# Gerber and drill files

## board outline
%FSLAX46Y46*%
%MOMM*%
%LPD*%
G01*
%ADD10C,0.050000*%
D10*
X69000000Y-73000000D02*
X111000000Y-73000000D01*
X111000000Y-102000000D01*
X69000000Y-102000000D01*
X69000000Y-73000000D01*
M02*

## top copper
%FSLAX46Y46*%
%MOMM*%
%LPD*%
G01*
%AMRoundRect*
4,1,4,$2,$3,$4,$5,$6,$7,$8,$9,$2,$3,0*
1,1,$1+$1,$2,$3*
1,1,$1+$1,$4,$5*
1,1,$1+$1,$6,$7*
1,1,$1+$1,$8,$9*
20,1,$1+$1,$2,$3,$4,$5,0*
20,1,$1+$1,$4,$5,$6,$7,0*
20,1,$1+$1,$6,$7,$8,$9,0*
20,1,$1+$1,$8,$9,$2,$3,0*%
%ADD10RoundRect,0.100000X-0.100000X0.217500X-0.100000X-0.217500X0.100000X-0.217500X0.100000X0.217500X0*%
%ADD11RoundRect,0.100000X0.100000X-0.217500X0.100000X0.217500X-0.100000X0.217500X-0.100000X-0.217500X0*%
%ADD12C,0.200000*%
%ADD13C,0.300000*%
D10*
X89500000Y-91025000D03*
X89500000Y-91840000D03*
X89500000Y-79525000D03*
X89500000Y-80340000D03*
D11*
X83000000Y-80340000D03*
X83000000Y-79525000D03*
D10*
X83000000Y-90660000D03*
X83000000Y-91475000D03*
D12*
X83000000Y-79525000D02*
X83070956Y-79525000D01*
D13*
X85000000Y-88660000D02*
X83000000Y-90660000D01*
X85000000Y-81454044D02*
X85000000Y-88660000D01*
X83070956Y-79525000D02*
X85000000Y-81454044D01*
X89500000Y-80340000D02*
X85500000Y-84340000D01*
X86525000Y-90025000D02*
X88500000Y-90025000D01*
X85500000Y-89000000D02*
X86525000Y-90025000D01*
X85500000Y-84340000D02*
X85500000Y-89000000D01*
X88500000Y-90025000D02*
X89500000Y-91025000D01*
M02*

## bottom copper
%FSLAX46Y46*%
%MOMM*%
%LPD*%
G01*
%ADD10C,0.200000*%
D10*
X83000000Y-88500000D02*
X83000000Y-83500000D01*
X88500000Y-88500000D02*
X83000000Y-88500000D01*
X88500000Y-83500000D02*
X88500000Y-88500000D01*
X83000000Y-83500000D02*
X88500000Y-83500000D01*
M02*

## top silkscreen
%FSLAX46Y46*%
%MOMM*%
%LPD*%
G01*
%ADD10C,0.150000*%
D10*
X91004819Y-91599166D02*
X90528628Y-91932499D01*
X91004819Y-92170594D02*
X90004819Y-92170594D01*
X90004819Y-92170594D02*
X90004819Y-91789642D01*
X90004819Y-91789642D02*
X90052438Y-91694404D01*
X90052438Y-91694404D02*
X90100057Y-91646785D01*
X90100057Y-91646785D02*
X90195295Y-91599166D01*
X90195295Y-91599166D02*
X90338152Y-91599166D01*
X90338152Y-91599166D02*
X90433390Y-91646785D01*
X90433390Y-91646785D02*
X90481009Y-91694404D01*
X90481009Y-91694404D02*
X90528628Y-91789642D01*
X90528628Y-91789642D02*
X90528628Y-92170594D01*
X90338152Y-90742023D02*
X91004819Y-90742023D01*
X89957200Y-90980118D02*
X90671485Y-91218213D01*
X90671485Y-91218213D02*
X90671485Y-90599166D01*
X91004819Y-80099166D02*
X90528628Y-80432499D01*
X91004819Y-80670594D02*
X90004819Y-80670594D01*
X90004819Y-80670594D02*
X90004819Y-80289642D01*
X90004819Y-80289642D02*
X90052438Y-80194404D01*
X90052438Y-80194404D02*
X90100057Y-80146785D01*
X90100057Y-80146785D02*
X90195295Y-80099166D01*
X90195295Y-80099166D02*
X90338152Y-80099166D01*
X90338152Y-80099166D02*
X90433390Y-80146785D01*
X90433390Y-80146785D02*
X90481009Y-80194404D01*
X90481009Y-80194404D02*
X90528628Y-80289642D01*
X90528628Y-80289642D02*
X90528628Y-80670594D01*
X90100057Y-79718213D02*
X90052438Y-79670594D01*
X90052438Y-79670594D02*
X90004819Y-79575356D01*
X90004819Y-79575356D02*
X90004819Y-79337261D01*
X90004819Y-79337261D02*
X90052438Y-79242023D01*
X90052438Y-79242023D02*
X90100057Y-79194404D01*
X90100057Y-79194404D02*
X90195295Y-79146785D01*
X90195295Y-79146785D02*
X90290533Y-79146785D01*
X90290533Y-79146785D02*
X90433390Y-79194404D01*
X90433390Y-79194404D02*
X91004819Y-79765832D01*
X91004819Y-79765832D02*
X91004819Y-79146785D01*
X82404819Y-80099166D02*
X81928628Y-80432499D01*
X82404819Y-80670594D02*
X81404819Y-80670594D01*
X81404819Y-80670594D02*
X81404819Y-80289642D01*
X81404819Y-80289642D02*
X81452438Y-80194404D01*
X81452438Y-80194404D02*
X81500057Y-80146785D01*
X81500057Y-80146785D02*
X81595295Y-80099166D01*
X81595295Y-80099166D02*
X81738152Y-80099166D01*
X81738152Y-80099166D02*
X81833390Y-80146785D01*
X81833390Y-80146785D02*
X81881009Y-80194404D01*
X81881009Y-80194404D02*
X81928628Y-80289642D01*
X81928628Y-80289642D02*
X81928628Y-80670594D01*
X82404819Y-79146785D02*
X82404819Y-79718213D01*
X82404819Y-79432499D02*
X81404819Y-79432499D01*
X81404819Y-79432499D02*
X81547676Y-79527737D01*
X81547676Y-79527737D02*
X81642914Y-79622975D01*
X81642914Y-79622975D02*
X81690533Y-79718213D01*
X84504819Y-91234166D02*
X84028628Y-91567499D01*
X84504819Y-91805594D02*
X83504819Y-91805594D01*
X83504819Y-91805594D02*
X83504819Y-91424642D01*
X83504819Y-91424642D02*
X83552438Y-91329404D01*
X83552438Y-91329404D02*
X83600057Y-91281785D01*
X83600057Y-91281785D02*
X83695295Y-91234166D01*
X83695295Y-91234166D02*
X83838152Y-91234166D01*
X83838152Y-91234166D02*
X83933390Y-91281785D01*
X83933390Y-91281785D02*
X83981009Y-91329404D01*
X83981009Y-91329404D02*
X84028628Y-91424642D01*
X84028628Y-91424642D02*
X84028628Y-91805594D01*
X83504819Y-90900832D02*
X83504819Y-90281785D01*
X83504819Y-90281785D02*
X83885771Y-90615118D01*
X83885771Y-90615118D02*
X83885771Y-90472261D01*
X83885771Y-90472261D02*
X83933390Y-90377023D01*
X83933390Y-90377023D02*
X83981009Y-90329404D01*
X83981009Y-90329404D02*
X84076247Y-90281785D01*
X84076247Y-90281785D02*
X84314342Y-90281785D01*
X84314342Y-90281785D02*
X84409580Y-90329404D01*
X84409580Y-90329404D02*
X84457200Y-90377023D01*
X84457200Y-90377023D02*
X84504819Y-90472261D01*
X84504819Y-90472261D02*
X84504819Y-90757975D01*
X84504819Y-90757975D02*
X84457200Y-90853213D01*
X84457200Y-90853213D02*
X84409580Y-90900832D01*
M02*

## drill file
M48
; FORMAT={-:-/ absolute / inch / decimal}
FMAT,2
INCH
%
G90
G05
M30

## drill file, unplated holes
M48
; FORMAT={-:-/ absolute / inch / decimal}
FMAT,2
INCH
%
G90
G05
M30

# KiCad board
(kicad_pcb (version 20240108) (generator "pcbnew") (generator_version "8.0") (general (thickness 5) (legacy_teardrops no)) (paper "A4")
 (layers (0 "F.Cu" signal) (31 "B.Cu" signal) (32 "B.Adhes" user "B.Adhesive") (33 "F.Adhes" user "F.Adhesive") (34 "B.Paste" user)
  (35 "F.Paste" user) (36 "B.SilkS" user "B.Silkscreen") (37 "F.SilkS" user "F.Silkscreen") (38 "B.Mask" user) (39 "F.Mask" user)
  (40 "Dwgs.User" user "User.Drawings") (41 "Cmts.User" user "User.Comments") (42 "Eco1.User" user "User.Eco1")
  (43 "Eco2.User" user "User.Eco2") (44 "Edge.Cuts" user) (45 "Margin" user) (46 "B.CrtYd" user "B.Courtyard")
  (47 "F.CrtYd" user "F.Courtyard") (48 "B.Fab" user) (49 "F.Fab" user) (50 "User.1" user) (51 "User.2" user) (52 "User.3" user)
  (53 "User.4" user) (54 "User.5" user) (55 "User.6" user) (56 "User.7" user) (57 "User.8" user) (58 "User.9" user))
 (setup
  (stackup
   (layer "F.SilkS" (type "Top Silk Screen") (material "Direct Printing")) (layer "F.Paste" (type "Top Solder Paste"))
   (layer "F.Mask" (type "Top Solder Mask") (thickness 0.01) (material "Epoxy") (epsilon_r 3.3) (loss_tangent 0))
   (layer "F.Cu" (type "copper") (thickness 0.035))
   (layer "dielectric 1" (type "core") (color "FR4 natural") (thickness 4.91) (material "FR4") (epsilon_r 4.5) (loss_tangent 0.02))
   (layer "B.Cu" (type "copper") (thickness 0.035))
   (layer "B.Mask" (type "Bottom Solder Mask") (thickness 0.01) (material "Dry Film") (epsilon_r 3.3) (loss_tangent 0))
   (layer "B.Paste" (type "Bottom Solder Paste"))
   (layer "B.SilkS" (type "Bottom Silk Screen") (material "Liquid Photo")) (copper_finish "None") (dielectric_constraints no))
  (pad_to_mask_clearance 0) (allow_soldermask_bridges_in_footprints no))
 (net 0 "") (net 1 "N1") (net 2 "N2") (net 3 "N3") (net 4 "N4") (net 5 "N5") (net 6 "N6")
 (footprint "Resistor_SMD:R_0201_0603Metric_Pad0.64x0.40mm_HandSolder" (layer "F.Cu") (at 89.5 91.4325 -90)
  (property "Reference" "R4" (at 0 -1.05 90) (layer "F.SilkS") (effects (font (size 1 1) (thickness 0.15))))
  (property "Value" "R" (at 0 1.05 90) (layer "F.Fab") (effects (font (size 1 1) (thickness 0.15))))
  (pad "" smd roundrect (at -0.4325 0 270) (size 0.458 0.36) (layers "F.Paste") (roundrect_rratio 0.25))
  (pad "" smd roundrect (at 0.4325 0 270) (size 0.458 0.36) (layers "F.Paste") (roundrect_rratio 0.25))
  (pad "1" smd roundrect (at -0.4075 0 270) (size 0.635 0.4) (layers "F.Cu" "F.Mask") (roundrect_rratio 0.25) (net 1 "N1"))
  (pad "2" smd roundrect (at 0.4075 0 270) (size 0.635 0.4) (layers "F.Cu" "F.Mask") (roundrect_rratio 0.25) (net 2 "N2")))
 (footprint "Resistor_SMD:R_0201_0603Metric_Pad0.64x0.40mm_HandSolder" (layer "F.Cu") (at 89.5 79.9325 -90)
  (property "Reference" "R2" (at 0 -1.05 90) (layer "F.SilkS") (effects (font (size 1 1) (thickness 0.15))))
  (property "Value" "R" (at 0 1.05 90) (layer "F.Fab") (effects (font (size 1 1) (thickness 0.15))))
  (pad "" smd roundrect (at -0.4325 0 270) (size 0.458 0.36) (layers "F.Paste") (roundrect_rratio 0.25))
  (pad "" smd roundrect (at 0.4325 0 270) (size 0.458 0.36) (layers "F.Paste") (roundrect_rratio 0.25))
  (pad "1" smd roundrect (at -0.4075 0 270) (size 0.635 0.4) (layers "F.Cu" "F.Mask") (roundrect_rratio 0.25) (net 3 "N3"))
  (pad "2" smd roundrect (at 0.4075 0 270) (size 0.635 0.4) (layers "F.Cu" "F.Mask") (roundrect_rratio 0.25) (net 1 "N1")))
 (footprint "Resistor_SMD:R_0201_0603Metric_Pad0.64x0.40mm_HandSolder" (layer "F.Cu") (at 83 79.9325 90)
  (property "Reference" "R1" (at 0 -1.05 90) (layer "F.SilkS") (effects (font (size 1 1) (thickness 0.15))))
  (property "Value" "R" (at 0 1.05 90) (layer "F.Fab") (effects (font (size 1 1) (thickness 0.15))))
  (pad "" smd roundrect (at -0.4325 0 90) (size 0.458 0.36) (layers "F.Paste") (roundrect_rratio 0.25))
  (pad "" smd roundrect (at 0.4325 0 90) (size 0.458 0.36) (layers "F.Paste") (roundrect_rratio 0.25))
  (pad "1" smd roundrect (at -0.4075 0 90) (size 0.635 0.4) (layers "F.Cu" "F.Mask") (roundrect_rratio 0.25) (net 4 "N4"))
  (pad "2" smd roundrect (at 0.4075 0 90) (size 0.635 0.4) (layers "F.Cu" "F.Mask") (roundrect_rratio 0.25) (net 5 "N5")))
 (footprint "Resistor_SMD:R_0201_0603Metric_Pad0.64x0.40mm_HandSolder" (layer "F.Cu") (at 83 91.0675 -90)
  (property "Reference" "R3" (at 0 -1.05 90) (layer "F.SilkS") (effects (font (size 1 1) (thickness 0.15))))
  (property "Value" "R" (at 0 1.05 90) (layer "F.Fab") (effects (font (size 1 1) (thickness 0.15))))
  (pad "" smd roundrect (at -0.4325 0 270) (size 0.458 0.36) (layers "F.Paste") (roundrect_rratio 0.25))
  (pad "" smd roundrect (at 0.4325 0 270) (size 0.458 0.36) (layers "F.Paste") (roundrect_rratio 0.25))
  (pad "1" smd roundrect (at -0.4075 0 270) (size 0.635 0.4) (layers "F.Cu" "F.Mask") (roundrect_rratio 0.25) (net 5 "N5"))
  (pad "2" smd roundrect (at 0.4075 0 270) (size 0.635 0.4) (layers "F.Cu" "F.Mask") (roundrect_rratio 0.25) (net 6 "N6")))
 (gr_line (start 88.5 88.5) (end 83 88.5) (stroke (width 0.2) (type default)) (layer "B.Cu"))
 (gr_line (start 83 88.5) (end 83 83.5) (stroke (width 0.2) (type default)) (layer "B.Cu"))
 (gr_line (start 88.5 83.5) (end 88.5 88.5) (stroke (width 0.2) (type default)) (layer "B.Cu"))
 (gr_line (start 83 83.5) (end 88.5 83.5) (stroke (width 0.2) (type default)) (layer "B.Cu"))
 (gr_rect (start 69 73) (end 111 102) (stroke (width 0.05) (type default)) (fill none) (layer "Edge.Cuts"))
 (segment (start 83 79.525) (end 83.070956 79.525) (width 0.2) (layer "F.Cu") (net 5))
 (segment (start 85 88.66) (end 83 90.66) (width 0.3) (layer "F.Cu") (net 5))
 (segment (start 85 81.454044) (end 85 88.66) (width 0.3) (layer "F.Cu") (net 5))
 (segment (start 83.070956 79.525) (end 85 81.454044) (width 0.3) (layer "F.Cu") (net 5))
 (segment (start 89.5 80.34) (end 85.5 84.34) (width 0.3) (layer "F.Cu") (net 1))
 (segment (start 86.525 90.025) (end 88.5 90.025) (width 0.3) (layer "F.Cu") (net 1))
 (segment (start 85.5 89) (end 86.525 90.025) (width 0.3) (layer "F.Cu") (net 1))
 (segment (start 85.5 84.34) (end 85.5 89) (width 0.3) (layer "F.Cu") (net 1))
 (segment (start 88.5 90.025) (end 89.5 91.025) (width 0.3) (layer "F.Cu") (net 1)))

